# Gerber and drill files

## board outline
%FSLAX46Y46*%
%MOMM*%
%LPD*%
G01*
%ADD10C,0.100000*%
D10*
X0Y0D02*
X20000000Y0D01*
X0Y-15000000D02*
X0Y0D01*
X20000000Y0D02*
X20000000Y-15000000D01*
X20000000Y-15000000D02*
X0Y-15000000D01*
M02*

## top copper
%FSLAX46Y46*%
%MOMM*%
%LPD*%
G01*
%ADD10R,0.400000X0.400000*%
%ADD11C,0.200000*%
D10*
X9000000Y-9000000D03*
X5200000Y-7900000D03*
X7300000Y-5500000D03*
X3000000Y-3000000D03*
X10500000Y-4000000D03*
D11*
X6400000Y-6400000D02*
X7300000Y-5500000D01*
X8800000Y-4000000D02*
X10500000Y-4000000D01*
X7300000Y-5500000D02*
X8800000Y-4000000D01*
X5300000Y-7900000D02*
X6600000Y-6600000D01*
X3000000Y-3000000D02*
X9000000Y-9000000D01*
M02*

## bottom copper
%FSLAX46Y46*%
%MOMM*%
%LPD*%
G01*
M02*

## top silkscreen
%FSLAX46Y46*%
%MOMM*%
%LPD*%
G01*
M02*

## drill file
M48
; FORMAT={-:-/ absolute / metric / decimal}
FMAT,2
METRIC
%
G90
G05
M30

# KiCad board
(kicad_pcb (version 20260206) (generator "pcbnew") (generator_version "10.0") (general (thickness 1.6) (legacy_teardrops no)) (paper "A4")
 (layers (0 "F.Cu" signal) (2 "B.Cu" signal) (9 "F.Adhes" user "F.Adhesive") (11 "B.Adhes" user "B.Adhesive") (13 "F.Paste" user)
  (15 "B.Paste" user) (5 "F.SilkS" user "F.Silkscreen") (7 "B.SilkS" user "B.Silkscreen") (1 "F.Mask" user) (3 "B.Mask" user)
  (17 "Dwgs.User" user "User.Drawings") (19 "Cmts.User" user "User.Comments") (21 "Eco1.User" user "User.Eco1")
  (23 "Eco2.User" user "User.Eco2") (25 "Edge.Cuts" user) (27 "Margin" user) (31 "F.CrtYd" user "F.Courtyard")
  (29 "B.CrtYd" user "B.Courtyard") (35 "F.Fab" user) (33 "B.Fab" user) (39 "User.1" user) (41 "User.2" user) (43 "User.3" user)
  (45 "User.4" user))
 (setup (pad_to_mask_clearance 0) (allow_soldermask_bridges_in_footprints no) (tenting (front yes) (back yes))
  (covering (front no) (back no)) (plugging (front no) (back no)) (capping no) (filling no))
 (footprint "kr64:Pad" (layer "F.Cu") (at 9 9)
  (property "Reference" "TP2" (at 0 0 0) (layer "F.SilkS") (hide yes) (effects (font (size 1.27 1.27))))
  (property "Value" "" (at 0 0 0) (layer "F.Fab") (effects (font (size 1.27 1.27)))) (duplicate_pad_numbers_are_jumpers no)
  (pad "1" smd rect (at 0 0) (size 0.4 0.4) (layers "F.Cu" "F.Mask" "F.Paste") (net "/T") (thermal_bridge_angle 45)))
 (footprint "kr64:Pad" (layer "F.Cu") (at 5.2 7.9)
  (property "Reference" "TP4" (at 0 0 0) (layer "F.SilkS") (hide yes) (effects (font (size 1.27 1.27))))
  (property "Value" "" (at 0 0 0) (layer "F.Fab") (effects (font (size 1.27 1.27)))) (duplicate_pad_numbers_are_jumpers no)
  (pad "1" smd rect (at 0 0) (size 0.4 0.4) (layers "F.Cu" "F.Mask" "F.Paste") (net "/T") (thermal_bridge_angle 45)))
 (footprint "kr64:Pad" (layer "F.Cu") (at 7.3 5.5)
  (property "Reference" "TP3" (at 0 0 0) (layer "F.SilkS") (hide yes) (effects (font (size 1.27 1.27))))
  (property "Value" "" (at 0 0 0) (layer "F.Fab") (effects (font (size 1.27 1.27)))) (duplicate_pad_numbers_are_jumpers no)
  (pad "1" smd rect (at 0 0) (size 0.4 0.4) (layers "F.Cu" "F.Mask" "F.Paste") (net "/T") (thermal_bridge_angle 45)))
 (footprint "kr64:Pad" (layer "F.Cu") (at 3 3)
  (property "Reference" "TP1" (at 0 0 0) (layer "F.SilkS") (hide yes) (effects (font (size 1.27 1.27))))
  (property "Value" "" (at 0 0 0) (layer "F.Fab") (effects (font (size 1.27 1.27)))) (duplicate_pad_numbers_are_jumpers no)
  (pad "1" smd rect (at 0 0) (size 0.4 0.4) (layers "F.Cu" "F.Mask" "F.Paste") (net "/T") (thermal_bridge_angle 45)))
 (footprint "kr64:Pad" (layer "F.Cu") (at 10.5 4)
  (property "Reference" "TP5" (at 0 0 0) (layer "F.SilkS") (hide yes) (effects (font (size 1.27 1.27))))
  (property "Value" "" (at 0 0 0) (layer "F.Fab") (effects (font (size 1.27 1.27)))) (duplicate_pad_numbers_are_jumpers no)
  (pad "1" smd rect (at 0 0) (size 0.4 0.4) (layers "F.Cu" "F.Mask" "F.Paste") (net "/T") (thermal_bridge_angle 45)))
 (gr_line (start 0 0) (end 20 0) (stroke (width 0.1) (type default)) (layer "Edge.Cuts"))
 (gr_line (start 0 15) (end 0 0) (stroke (width 0.1) (type default)) (layer "Edge.Cuts"))
 (gr_line (start 20 0) (end 20 15) (stroke (width 0.1) (type default)) (layer "Edge.Cuts"))
 (gr_line (start 20 15) (end 0 15) (stroke (width 0.1) (type default)) (layer "Edge.Cuts"))
 (segment (start 6.4 6.4) (end 7.3 5.5) (width 0.2) (layer "F.Cu") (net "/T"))
 (segment (start 8.8 4) (end 10.5 4) (width 0.2) (layer "F.Cu") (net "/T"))
 (segment (start 7.3 5.5) (end 8.8 4) (width 0.2) (layer "F.Cu") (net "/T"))
 (segment (start 5.3 7.9) (end 6.6 6.6) (width 0.2) (layer "F.Cu") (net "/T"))
 (segment (start 3 3) (end 9 9) (width 0.2) (layer "F.Cu") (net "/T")))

